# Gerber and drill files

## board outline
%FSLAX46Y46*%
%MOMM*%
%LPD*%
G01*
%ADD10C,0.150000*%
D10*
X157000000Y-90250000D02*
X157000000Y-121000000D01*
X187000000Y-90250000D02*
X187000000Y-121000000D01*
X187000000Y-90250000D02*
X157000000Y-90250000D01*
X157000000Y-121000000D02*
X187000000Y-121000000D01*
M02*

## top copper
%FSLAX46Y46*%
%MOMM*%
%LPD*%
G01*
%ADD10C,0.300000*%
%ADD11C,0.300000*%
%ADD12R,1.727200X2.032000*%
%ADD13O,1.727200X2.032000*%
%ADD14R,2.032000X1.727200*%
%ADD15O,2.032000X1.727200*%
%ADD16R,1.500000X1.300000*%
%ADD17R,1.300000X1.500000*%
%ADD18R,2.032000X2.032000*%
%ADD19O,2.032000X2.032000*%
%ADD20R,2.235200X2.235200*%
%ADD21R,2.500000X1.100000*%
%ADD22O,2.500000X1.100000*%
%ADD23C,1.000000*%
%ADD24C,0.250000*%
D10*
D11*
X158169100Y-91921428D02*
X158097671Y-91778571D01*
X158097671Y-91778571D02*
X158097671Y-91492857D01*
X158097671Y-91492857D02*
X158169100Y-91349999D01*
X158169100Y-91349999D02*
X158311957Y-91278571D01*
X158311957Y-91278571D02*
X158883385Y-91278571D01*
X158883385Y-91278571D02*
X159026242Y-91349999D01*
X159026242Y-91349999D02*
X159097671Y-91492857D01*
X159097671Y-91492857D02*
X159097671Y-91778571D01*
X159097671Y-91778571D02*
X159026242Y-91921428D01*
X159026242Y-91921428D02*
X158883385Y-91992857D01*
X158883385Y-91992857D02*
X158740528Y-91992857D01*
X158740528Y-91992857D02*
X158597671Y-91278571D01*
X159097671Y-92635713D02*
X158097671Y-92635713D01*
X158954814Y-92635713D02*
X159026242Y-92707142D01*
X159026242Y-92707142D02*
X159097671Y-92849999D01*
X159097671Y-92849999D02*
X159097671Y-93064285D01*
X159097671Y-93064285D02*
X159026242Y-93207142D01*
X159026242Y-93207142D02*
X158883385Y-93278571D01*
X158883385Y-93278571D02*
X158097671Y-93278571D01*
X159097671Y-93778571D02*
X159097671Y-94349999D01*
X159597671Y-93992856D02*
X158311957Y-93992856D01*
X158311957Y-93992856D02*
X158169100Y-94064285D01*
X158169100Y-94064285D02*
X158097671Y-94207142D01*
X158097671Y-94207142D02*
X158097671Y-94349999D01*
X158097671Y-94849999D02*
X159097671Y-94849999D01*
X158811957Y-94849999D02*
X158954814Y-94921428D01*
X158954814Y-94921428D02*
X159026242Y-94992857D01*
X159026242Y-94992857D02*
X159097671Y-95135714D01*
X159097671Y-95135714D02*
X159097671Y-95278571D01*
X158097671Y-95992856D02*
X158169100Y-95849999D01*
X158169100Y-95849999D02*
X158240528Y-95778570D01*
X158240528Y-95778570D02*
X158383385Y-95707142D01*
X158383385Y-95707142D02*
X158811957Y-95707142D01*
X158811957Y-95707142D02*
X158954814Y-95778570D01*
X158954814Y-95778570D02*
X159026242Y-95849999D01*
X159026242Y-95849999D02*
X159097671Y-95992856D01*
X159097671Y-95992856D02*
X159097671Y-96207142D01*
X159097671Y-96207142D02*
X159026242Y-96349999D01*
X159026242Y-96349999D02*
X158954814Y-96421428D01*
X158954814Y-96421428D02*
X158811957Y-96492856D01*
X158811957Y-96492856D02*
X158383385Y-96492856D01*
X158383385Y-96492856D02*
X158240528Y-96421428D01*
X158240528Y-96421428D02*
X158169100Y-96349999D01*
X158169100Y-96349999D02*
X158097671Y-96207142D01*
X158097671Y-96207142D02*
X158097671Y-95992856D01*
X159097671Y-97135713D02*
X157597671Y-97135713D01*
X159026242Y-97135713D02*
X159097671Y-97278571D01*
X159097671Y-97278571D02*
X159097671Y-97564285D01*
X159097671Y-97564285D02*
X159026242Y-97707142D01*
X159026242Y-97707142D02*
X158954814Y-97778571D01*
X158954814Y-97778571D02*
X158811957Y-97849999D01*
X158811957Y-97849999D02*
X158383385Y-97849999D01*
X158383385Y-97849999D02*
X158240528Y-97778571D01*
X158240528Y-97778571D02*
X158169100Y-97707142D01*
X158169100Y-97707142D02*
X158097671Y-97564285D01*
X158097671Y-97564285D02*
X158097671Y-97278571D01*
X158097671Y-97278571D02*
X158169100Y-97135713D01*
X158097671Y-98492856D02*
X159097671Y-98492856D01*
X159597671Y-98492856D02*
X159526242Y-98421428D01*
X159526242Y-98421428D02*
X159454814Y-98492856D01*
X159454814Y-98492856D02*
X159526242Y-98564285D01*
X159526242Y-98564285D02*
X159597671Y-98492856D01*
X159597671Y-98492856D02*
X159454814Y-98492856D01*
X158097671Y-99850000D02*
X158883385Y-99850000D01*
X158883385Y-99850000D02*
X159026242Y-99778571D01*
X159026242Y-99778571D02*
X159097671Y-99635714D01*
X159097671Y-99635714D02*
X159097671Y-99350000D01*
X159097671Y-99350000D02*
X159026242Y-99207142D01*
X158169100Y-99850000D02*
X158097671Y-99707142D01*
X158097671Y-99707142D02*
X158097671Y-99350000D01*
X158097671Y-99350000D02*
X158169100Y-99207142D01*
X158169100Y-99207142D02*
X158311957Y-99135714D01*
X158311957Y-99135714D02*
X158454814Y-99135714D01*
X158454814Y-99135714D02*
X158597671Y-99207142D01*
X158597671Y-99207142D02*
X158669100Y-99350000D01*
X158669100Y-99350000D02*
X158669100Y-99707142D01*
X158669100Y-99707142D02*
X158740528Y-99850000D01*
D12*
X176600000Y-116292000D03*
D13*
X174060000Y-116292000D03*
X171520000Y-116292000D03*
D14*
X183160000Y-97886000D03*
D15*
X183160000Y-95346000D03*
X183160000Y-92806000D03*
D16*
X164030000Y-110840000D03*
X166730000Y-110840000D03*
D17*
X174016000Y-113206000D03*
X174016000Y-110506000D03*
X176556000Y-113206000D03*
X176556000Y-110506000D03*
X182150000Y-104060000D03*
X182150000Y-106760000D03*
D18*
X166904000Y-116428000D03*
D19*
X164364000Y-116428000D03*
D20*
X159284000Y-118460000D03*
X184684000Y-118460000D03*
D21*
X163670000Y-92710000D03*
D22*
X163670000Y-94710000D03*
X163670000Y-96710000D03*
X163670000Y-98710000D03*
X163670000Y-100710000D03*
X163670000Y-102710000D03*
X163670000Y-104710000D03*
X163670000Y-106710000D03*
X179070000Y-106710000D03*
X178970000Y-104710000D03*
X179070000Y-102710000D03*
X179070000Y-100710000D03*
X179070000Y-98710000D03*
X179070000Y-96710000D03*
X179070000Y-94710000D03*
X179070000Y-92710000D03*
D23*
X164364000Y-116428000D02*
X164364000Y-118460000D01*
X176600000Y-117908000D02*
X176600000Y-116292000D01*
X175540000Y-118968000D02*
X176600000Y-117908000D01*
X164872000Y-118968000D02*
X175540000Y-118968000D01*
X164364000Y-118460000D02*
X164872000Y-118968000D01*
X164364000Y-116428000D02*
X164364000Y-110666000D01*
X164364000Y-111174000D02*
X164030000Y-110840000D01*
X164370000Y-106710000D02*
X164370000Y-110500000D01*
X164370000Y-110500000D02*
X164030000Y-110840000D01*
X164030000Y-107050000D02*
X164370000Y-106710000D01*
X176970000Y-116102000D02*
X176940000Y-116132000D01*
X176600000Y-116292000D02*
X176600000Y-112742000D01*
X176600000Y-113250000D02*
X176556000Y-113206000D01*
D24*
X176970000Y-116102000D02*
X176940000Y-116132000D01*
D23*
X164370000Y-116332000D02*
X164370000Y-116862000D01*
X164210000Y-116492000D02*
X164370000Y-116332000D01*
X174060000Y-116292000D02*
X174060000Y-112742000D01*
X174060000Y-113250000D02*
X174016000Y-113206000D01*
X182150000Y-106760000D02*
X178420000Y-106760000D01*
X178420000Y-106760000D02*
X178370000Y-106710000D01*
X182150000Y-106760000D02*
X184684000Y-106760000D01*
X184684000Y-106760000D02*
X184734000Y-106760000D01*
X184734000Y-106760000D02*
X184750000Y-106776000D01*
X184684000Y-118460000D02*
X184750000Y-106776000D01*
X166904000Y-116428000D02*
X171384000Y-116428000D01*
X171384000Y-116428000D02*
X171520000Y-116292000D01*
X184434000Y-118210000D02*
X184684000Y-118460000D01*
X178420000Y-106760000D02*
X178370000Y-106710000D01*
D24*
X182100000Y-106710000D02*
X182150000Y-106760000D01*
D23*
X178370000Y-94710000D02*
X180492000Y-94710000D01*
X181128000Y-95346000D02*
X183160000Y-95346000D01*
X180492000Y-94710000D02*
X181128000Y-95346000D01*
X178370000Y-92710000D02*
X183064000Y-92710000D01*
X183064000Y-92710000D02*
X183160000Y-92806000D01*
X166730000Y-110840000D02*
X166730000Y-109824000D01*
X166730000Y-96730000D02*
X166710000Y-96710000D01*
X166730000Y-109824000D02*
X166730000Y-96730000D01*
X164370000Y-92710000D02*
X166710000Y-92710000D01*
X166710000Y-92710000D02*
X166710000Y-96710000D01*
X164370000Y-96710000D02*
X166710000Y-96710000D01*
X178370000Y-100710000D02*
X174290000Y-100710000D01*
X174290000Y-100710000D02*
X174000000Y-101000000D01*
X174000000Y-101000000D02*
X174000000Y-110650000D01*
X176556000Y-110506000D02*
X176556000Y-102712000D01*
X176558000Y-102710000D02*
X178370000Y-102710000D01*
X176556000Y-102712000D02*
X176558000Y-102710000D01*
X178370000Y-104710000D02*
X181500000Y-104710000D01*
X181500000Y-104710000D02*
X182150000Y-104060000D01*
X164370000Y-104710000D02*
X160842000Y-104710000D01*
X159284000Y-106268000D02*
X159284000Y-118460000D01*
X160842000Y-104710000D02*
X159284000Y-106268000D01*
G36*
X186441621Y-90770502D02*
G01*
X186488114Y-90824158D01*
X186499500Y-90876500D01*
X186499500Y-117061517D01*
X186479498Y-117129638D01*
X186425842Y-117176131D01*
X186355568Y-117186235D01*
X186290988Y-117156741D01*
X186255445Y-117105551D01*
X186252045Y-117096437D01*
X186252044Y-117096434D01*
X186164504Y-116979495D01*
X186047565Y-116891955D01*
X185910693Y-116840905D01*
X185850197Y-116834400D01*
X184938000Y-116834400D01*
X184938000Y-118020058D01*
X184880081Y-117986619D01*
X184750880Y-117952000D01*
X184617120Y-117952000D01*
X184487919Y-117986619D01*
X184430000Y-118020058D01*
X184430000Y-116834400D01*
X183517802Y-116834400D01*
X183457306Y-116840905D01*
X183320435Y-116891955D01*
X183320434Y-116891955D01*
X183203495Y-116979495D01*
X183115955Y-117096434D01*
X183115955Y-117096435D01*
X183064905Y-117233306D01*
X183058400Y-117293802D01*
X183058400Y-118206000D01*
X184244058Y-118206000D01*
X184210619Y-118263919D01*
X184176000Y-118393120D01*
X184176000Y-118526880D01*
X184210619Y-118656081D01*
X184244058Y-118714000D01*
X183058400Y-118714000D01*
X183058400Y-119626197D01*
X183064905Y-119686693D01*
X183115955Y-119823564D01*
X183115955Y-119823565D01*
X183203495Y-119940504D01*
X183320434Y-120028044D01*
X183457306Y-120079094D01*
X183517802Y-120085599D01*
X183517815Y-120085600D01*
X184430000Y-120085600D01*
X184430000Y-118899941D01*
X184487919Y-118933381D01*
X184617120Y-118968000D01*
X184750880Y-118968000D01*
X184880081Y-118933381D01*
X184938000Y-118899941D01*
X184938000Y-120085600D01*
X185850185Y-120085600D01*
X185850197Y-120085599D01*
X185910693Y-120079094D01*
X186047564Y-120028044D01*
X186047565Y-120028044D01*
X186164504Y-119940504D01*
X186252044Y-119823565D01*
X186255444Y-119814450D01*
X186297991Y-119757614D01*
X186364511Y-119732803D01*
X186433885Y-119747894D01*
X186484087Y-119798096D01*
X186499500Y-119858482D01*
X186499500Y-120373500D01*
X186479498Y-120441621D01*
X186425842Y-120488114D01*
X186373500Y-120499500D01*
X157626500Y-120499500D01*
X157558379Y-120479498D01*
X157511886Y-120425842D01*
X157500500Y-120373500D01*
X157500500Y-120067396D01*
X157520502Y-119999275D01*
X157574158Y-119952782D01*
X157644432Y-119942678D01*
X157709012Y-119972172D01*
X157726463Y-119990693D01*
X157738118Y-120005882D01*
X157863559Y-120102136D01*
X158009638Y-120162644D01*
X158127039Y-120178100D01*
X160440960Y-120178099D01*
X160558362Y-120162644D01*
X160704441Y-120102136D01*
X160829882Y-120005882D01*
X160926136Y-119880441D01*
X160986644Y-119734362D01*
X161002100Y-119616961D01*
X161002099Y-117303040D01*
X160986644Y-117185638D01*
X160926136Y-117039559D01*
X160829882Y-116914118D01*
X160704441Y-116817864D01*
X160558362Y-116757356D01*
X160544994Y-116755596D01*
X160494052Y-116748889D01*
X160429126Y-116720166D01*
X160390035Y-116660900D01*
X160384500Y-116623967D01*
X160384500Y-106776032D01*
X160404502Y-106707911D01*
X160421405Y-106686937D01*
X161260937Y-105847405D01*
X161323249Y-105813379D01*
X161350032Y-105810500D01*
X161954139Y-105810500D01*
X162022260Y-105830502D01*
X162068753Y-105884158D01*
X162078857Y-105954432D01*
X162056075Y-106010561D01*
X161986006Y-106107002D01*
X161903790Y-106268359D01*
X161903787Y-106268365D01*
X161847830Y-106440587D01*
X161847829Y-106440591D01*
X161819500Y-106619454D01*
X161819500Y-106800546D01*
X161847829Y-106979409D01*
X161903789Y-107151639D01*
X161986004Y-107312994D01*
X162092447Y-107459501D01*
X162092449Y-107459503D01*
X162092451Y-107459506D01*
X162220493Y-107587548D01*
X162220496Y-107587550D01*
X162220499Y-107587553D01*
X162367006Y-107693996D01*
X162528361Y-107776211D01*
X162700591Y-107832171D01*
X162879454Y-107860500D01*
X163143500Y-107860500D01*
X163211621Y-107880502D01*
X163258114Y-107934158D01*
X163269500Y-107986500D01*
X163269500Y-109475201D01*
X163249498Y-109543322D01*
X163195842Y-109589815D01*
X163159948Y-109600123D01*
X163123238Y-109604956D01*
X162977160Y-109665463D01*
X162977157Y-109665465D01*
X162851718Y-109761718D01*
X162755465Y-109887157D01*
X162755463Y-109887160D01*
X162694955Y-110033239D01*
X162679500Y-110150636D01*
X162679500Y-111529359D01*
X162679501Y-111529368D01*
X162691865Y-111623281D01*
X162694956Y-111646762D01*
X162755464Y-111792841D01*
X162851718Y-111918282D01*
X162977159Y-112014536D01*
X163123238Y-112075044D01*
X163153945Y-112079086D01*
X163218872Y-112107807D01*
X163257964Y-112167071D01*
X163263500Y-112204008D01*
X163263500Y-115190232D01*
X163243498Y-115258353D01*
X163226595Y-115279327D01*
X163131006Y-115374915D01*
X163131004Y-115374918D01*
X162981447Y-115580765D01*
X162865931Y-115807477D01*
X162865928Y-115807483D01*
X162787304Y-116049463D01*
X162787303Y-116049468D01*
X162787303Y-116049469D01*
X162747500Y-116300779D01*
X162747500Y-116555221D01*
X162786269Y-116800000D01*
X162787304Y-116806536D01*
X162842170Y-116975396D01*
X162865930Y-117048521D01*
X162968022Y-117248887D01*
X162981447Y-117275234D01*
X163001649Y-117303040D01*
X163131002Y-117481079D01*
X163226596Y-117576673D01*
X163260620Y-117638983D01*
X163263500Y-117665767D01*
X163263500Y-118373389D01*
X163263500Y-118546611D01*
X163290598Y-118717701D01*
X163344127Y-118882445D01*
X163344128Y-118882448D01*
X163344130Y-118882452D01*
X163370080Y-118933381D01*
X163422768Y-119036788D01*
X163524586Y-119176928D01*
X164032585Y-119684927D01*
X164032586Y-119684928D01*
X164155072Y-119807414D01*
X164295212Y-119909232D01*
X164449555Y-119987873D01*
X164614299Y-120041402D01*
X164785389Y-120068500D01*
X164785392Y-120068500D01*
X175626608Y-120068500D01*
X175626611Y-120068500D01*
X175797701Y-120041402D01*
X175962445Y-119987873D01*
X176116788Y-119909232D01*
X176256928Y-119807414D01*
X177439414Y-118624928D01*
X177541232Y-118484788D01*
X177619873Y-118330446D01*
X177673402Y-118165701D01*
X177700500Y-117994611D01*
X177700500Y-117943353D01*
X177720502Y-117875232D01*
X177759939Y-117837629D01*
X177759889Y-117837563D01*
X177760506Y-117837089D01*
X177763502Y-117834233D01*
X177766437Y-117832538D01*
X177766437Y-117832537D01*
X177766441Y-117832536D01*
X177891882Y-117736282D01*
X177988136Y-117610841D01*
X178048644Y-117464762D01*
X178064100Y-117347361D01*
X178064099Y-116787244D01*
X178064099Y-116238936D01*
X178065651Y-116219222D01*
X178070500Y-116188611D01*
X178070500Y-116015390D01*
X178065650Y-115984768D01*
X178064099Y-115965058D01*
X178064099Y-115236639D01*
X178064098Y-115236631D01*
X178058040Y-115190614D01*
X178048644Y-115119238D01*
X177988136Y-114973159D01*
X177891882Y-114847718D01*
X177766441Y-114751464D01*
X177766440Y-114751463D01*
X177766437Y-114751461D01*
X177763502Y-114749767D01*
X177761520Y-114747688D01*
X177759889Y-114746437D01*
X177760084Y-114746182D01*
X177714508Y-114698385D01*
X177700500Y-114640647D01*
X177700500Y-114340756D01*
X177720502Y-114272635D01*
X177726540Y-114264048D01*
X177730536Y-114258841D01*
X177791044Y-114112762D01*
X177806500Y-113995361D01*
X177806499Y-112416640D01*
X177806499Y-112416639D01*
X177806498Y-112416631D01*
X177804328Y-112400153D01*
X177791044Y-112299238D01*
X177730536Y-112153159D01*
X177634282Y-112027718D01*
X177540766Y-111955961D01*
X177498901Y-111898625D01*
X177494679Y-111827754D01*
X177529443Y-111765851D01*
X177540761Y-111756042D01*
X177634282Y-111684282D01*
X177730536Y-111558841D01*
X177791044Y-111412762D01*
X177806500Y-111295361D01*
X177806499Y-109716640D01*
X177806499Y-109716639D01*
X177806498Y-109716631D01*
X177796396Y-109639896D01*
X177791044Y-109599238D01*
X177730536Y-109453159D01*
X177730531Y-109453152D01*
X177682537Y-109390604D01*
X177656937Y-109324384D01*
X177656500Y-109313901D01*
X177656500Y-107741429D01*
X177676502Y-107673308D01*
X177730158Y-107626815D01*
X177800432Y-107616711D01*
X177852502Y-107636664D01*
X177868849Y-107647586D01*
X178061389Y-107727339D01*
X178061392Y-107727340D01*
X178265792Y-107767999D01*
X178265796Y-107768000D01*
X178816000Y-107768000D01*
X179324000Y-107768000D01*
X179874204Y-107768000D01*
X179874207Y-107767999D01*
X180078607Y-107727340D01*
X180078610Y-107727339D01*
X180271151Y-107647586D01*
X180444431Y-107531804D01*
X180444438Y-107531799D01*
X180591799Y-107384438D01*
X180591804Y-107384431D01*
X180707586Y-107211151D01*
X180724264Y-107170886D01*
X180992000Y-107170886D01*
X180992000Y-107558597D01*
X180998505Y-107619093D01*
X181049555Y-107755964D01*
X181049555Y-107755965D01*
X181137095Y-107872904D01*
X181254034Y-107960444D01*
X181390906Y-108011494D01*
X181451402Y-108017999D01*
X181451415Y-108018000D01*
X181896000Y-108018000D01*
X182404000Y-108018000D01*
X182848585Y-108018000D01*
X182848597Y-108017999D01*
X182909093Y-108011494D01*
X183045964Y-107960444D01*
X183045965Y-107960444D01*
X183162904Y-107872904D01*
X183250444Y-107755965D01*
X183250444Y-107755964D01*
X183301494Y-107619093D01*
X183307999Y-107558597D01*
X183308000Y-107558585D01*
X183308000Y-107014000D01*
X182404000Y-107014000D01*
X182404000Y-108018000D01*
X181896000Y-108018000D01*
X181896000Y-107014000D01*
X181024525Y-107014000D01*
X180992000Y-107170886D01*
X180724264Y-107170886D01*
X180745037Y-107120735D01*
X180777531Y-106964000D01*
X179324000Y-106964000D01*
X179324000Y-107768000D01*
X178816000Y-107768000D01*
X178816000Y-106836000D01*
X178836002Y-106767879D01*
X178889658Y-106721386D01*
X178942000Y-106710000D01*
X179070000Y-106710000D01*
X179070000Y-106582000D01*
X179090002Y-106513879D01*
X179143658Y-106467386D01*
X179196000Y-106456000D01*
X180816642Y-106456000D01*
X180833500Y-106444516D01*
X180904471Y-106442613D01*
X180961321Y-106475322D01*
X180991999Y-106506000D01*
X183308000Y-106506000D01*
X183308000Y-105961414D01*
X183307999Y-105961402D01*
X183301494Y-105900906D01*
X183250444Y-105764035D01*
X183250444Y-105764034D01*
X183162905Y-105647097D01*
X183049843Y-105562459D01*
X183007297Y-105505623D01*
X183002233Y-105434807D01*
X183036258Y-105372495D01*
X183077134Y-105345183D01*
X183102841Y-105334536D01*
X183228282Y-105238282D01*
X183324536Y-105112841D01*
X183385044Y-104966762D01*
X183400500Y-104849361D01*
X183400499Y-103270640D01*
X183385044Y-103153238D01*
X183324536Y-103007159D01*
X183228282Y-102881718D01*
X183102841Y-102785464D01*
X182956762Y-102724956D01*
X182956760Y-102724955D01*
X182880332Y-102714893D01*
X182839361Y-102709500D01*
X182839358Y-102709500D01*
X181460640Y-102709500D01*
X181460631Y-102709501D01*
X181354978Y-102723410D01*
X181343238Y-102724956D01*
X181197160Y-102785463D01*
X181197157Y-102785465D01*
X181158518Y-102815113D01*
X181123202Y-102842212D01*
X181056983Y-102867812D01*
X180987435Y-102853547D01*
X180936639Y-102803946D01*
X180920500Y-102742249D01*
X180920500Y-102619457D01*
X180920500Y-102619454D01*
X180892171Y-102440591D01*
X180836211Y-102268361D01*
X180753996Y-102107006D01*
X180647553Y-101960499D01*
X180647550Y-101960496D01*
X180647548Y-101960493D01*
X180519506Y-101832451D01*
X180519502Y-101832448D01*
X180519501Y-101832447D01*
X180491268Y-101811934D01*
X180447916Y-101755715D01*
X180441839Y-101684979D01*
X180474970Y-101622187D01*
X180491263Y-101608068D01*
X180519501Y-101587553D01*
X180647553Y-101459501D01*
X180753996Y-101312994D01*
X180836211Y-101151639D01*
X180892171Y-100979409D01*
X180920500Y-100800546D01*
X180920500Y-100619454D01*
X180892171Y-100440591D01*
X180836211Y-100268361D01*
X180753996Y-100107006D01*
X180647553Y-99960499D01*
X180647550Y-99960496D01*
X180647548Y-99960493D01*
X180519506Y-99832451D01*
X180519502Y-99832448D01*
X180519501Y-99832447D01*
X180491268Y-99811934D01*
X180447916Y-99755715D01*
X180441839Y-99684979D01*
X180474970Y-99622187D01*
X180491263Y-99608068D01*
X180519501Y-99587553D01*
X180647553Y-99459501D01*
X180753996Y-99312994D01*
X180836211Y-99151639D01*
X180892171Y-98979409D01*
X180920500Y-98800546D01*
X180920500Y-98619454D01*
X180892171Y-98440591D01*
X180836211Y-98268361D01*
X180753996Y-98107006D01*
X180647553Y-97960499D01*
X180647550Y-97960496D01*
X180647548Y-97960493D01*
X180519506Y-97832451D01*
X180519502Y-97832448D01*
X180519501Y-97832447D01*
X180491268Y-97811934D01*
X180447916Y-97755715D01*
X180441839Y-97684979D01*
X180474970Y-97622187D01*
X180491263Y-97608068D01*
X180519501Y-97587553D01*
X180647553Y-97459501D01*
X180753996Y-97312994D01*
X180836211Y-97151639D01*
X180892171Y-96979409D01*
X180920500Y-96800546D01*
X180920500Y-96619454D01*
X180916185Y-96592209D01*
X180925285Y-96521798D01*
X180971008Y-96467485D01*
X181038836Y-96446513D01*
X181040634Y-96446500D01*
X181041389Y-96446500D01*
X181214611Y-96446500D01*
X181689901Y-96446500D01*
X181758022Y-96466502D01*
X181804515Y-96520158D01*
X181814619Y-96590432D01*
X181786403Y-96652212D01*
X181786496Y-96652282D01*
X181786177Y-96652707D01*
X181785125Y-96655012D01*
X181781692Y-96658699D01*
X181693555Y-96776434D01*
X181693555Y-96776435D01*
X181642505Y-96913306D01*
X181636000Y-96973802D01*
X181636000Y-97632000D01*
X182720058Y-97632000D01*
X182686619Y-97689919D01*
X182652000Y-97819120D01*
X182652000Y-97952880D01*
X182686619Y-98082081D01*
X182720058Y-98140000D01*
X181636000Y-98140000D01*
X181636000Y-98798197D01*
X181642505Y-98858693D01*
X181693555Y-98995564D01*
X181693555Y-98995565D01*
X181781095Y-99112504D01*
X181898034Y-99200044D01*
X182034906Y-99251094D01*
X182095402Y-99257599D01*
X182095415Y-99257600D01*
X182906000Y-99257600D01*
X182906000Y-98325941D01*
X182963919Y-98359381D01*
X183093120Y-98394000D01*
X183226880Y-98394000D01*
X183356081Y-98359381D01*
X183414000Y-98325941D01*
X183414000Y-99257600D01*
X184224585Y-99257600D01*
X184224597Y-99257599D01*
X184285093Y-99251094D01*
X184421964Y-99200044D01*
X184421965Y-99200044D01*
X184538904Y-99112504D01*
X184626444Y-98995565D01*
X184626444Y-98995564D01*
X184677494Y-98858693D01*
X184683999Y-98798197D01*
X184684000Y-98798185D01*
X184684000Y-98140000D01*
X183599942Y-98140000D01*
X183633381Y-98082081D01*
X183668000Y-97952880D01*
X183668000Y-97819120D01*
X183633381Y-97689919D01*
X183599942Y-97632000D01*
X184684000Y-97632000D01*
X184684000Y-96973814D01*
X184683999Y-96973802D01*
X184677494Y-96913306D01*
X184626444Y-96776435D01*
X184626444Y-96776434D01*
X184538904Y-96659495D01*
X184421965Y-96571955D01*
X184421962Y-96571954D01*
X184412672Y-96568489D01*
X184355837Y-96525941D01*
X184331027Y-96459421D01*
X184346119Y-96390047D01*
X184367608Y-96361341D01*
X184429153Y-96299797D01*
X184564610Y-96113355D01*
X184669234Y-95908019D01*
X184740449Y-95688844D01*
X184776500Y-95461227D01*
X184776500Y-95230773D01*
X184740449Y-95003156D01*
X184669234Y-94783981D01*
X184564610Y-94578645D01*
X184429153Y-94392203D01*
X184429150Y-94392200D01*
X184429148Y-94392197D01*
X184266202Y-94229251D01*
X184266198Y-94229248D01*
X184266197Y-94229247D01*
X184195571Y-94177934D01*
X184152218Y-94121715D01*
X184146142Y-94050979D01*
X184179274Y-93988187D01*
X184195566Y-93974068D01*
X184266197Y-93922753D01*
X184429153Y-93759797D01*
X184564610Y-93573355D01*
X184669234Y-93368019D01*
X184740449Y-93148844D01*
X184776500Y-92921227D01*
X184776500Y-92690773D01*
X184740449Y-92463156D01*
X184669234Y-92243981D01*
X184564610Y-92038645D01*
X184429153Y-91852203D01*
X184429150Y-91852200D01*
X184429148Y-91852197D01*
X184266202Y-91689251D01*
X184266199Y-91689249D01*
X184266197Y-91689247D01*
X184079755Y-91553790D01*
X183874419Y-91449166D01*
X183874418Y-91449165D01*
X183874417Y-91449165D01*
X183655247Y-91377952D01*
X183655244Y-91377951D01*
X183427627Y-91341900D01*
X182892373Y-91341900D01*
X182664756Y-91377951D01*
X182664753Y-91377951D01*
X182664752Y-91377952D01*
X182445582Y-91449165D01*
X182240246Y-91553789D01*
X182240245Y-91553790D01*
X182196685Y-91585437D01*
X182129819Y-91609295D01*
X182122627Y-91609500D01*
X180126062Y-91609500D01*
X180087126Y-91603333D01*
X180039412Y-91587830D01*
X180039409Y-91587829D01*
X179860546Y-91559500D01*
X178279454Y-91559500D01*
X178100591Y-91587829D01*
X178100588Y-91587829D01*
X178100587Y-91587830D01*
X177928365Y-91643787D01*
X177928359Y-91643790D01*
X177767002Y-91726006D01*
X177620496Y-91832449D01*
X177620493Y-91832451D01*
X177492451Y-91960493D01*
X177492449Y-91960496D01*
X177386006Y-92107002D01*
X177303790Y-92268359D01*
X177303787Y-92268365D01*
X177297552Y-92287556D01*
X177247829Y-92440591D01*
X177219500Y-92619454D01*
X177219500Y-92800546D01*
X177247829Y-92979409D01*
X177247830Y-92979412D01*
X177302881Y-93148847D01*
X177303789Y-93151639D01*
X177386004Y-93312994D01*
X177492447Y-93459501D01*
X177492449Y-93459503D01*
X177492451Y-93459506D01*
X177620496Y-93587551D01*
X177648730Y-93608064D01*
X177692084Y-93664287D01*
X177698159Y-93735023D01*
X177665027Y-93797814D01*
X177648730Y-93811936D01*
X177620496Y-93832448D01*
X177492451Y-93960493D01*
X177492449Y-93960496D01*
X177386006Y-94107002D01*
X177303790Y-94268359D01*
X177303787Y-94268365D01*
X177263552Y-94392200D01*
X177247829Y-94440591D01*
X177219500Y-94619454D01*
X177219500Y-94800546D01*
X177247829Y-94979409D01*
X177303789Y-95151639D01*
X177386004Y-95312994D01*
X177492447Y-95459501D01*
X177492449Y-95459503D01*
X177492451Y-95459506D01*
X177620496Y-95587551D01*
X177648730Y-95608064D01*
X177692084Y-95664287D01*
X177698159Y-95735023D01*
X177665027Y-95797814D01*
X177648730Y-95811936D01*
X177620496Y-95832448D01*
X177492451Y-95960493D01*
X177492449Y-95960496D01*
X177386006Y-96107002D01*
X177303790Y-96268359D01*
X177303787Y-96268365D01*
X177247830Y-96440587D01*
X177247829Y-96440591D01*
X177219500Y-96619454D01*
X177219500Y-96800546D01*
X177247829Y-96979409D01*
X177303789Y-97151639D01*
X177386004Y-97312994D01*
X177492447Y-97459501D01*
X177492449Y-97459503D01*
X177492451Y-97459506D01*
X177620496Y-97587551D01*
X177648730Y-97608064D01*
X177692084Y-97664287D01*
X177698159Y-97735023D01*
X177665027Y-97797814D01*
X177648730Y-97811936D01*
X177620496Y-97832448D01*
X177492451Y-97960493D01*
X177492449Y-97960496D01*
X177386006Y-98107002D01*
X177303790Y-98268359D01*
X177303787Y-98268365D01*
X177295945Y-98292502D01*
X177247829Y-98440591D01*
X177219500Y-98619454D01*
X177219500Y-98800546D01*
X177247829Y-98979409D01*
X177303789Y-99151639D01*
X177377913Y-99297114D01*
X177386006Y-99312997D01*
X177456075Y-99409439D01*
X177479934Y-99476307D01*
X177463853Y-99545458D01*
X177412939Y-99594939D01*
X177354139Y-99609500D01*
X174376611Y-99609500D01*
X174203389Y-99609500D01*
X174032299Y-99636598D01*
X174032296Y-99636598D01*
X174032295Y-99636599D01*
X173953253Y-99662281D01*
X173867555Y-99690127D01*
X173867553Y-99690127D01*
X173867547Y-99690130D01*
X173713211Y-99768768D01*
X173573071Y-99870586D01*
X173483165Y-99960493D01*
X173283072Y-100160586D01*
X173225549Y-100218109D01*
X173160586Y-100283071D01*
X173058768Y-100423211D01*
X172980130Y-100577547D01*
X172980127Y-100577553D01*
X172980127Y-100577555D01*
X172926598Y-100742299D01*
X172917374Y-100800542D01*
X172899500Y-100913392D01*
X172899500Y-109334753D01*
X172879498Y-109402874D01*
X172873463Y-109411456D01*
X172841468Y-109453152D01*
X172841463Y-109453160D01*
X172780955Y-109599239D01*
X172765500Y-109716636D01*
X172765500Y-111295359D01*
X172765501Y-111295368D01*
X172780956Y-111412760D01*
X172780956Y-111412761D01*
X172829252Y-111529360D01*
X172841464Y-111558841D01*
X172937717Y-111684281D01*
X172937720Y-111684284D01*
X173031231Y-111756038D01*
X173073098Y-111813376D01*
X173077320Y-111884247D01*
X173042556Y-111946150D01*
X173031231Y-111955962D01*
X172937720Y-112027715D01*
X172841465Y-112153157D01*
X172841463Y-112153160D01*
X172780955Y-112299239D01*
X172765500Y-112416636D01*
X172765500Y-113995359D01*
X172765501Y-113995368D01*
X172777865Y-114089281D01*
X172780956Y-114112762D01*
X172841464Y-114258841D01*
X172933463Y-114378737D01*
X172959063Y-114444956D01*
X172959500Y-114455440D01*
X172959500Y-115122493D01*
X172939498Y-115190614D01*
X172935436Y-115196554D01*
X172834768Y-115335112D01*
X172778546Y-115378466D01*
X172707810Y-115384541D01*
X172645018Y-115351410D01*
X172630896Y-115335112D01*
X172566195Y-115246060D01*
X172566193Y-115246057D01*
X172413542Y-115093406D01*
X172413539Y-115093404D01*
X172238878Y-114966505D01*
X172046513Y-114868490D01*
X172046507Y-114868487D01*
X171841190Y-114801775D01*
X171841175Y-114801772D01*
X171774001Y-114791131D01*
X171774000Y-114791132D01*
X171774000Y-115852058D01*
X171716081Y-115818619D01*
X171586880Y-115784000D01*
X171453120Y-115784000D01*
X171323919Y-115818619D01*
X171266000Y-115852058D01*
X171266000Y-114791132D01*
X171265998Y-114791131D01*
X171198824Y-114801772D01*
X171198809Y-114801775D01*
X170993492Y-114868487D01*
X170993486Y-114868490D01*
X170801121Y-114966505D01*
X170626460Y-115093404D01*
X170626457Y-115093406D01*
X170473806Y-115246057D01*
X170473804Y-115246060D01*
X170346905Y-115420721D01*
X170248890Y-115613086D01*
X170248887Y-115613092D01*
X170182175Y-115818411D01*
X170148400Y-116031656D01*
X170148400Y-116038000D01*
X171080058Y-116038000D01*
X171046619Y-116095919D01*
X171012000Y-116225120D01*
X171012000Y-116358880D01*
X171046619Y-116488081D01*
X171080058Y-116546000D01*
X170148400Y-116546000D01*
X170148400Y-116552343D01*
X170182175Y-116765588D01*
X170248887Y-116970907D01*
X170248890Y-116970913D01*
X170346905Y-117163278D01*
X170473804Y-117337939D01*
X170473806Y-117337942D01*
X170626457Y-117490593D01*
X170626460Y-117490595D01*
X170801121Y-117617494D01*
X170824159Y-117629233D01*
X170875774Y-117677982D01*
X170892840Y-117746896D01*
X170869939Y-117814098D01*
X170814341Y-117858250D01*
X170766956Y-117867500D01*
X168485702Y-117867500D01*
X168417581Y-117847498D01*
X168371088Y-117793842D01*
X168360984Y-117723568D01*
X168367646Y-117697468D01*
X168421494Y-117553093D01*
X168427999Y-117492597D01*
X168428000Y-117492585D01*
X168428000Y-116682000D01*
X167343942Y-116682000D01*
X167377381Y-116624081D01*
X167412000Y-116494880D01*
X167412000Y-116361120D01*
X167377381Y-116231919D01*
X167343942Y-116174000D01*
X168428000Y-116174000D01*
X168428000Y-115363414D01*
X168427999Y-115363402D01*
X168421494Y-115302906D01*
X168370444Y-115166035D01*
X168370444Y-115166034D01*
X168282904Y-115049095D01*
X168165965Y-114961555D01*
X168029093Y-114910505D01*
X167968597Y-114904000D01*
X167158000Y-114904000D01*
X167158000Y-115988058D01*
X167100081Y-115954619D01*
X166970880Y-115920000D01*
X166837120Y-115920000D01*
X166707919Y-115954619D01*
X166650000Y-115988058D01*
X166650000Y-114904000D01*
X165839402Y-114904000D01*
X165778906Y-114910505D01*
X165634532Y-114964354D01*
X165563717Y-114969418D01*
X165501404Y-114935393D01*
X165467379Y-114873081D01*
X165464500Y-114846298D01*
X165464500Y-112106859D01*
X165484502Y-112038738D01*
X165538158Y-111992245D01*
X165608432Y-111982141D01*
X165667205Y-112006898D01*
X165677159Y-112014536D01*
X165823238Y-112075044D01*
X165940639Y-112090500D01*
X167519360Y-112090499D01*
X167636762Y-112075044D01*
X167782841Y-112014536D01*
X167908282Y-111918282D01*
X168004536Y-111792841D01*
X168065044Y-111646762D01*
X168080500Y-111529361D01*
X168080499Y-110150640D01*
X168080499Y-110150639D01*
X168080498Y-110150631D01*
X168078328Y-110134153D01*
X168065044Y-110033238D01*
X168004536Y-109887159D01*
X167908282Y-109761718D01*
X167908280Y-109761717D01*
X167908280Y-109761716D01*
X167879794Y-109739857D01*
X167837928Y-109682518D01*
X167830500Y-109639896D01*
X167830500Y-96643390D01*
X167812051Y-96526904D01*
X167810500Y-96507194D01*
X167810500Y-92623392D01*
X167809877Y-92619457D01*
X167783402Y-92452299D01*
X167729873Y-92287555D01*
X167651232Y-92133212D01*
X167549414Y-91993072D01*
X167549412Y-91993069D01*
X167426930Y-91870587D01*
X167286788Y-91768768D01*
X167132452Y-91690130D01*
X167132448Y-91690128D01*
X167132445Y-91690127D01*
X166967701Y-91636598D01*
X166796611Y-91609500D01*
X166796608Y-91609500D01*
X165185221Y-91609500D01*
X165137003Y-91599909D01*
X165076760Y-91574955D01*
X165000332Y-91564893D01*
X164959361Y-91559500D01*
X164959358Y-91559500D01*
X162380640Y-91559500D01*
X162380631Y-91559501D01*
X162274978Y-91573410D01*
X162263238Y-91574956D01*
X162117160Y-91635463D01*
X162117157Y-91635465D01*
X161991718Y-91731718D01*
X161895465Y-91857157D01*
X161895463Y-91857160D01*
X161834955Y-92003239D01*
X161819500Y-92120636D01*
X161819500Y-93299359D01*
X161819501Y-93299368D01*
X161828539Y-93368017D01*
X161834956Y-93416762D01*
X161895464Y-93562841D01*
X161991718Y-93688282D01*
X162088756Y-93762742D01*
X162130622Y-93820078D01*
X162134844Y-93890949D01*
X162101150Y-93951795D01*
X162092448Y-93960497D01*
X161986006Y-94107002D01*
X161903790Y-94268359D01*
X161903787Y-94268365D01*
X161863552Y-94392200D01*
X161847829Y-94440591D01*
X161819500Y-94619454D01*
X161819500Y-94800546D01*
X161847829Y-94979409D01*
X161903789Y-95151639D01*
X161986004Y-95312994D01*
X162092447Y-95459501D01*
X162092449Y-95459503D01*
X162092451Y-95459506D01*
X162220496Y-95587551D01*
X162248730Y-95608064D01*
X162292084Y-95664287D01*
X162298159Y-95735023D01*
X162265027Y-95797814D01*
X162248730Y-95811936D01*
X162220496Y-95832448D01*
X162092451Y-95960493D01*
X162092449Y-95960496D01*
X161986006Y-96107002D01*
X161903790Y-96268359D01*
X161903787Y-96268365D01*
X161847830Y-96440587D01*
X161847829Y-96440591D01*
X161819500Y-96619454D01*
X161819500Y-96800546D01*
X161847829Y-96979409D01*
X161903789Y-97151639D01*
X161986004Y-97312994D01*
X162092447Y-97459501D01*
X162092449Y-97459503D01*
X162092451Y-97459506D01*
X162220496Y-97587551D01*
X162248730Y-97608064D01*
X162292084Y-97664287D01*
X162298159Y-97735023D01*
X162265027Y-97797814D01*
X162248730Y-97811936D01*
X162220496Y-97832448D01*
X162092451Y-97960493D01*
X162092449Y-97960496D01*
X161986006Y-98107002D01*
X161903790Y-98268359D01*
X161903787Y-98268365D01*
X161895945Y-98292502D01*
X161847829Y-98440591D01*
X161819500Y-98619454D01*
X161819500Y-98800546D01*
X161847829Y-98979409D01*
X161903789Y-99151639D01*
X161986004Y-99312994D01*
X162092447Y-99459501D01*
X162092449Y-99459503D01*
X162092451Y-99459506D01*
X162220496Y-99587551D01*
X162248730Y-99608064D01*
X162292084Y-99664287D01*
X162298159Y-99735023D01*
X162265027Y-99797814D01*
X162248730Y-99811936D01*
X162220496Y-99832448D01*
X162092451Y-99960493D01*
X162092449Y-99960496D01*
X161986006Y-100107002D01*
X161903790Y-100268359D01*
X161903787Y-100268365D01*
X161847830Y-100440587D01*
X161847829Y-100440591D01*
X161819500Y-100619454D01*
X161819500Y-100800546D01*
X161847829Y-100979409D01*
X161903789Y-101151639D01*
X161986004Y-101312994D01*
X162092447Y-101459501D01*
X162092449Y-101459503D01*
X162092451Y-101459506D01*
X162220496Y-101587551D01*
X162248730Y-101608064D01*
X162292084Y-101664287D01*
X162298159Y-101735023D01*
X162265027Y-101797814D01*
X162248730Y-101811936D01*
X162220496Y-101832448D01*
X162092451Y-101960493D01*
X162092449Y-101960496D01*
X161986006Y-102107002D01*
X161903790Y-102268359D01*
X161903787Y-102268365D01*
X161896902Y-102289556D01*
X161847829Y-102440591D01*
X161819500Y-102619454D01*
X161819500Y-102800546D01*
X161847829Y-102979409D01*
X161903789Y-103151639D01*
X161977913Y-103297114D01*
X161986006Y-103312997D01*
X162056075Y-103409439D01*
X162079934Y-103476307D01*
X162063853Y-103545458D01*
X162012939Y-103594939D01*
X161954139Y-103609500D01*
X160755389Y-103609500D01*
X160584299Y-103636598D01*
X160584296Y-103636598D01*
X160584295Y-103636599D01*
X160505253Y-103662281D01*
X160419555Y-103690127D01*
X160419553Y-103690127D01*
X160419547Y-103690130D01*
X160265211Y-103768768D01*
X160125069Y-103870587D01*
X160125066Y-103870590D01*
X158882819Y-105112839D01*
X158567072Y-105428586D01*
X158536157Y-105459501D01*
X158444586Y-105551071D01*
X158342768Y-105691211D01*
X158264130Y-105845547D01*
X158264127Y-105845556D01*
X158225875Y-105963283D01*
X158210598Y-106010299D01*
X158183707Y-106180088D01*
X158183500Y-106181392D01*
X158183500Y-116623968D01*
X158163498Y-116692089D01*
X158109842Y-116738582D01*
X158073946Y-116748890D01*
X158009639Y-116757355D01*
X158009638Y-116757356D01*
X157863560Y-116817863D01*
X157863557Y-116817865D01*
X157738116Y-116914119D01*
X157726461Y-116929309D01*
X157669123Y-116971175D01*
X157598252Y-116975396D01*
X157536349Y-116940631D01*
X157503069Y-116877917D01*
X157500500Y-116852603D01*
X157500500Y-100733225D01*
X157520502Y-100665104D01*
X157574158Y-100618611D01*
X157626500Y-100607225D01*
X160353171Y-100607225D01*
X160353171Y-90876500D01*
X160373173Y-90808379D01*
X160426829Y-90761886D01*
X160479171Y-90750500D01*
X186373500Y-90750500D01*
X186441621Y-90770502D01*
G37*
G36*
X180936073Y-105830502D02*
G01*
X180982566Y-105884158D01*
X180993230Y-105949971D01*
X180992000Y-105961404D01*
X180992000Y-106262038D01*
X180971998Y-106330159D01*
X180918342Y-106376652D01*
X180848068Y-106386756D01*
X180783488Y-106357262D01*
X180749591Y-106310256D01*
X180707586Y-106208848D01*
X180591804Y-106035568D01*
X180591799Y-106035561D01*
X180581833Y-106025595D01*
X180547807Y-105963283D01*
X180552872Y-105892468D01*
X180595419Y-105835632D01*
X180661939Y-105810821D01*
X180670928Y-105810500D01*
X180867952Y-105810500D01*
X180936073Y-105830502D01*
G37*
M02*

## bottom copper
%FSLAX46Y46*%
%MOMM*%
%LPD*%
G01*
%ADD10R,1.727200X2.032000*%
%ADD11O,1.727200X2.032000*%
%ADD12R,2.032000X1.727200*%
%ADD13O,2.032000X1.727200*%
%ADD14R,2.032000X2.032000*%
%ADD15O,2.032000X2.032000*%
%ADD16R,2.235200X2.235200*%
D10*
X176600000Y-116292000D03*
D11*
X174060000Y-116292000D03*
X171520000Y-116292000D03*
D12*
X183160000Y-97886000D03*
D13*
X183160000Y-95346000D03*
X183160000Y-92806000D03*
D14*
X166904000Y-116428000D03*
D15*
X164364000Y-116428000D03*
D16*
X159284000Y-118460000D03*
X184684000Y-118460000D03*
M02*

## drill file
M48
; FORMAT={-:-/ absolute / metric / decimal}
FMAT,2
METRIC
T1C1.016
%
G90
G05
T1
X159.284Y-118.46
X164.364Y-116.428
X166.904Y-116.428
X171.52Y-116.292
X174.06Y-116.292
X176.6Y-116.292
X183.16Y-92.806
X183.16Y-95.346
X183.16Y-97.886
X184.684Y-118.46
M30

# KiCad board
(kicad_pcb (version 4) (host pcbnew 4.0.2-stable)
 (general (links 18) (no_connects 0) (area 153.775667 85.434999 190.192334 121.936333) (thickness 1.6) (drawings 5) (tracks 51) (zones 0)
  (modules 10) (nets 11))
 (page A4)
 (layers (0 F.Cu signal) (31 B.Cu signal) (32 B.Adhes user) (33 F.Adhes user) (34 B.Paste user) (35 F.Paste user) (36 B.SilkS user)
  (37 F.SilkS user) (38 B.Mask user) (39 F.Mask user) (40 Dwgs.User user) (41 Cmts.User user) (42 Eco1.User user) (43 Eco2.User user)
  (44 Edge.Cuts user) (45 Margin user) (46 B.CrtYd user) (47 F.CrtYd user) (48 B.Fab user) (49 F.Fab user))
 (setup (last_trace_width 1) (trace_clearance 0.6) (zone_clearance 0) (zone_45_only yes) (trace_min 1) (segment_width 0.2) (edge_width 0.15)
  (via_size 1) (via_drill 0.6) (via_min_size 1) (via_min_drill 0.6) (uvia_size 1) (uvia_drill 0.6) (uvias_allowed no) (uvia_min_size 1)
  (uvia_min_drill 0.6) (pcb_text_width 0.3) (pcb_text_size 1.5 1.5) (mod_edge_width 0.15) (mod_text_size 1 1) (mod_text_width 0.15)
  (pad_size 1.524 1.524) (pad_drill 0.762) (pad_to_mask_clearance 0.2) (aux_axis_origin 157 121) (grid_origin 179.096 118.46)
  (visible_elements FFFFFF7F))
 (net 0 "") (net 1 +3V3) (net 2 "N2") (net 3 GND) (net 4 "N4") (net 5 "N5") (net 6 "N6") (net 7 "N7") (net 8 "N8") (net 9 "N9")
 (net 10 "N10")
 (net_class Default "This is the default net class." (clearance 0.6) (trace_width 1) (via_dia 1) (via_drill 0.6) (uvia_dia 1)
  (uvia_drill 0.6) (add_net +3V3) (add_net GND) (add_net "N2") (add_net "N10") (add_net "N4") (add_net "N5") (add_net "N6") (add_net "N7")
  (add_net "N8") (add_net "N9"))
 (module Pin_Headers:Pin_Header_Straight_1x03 (layer F.Cu) (at 176.6 116.292 270)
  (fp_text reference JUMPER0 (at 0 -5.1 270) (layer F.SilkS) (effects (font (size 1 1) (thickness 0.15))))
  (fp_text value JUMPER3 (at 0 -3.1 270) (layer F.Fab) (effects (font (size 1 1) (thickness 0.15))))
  (pad 1 thru_hole rect (at 0 0 270) (size 2.032 1.7272) (drill 1.016) (layers *.Cu *.Mask F.SilkS) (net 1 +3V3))
  (pad 2 thru_hole oval (at 0 2.54 270) (size 2.032 1.7272) (drill 1.016) (layers *.Cu *.Mask F.SilkS) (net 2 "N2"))
  (pad 3 thru_hole oval (at 0 5.08 270) (size 2.032 1.7272) (drill 1.016) (layers *.Cu *.Mask F.SilkS) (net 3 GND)))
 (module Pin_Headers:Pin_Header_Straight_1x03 (layer F.Cu) (at 183.16 97.886 180)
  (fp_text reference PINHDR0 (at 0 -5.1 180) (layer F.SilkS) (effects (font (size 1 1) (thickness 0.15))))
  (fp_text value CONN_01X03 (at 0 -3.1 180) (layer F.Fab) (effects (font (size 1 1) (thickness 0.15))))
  (pad 1 thru_hole rect (at 0 0 180) (size 2.032 1.7272) (drill 1.016) (layers *.Cu *.Mask F.SilkS) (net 3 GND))
  (pad 2 thru_hole oval (at 0 2.54 180) (size 2.032 1.7272) (drill 1.016) (layers *.Cu *.Mask F.SilkS) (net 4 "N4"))
  (pad 3 thru_hole oval (at 0 5.08 180) (size 2.032 1.7272) (drill 1.016) (layers *.Cu *.Mask F.SilkS) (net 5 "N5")))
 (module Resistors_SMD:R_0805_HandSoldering (layer F.Cu) (at 165.38 110.84)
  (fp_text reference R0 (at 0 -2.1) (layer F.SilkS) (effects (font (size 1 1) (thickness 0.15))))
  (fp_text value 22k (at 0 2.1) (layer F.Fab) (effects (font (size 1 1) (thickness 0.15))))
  (pad 1 smd rect (at -1.35 0) (size 1.5 1.3) (layers F.Cu F.Paste F.Mask) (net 1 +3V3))
  (pad 2 smd rect (at 1.35 0) (size 1.5 1.3) (layers F.Cu F.Paste F.Mask) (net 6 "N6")))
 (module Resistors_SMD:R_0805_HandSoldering (layer F.Cu) (at 174.016 111.856 90)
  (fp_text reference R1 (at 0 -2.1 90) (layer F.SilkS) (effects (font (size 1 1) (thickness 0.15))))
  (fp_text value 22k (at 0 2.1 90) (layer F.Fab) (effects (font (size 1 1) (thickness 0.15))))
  (pad 1 smd rect (at -1.35 0 90) (size 1.5 1.3) (layers F.Cu F.Paste F.Mask) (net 2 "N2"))
  (pad 2 smd rect (at 1.35 0 90) (size 1.5 1.3) (layers F.Cu F.Paste F.Mask) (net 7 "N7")))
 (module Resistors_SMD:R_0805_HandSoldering (layer F.Cu) (at 176.556 111.856 90)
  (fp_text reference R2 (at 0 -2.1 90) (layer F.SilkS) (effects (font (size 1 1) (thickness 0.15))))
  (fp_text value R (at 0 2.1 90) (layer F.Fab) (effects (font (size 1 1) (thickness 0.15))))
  (pad 1 smd rect (at -1.35 0 90) (size 1.5 1.3) (layers F.Cu F.Paste F.Mask) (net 1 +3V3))
  (pad 2 smd rect (at 1.35 0 90) (size 1.5 1.3) (layers F.Cu F.Paste F.Mask) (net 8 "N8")))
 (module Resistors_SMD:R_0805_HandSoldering (layer F.Cu) (at 182.15 105.41 270)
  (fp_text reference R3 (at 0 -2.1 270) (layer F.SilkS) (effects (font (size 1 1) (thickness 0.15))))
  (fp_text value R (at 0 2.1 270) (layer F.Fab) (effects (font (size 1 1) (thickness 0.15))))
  (pad 1 smd rect (at -1.35 0 270) (size 1.5 1.3) (layers F.Cu F.Paste F.Mask) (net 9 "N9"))
  (pad 2 smd rect (at 1.35 0 270) (size 1.5 1.3) (layers F.Cu F.Paste F.Mask) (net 3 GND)))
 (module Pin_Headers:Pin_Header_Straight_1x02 (layer F.Cu) (at 166.904 116.428 270)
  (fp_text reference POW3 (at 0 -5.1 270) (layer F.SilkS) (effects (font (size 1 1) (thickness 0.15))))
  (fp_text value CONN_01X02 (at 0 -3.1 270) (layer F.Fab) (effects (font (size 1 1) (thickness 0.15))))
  (pad 1 thru_hole rect (at 0 0 270) (size 2.032 2.032) (drill 1.016) (layers *.Cu *.Mask F.SilkS) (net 3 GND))
  (pad 2 thru_hole oval (at 0 2.54 270) (size 2.032 2.032) (drill 1.016) (layers *.Cu *.Mask F.SilkS) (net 1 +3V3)))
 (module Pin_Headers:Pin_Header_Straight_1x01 (layer F.Cu) (at 159.284 118.46)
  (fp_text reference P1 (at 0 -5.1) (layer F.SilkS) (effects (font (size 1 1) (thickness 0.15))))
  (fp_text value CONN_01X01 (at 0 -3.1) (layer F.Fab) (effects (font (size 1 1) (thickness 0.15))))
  (pad 1 thru_hole rect (at 0 0) (size 2.2352 2.2352) (drill 1.016) (layers *.Cu *.Mask F.SilkS) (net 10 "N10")))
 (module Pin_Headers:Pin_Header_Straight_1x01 (layer F.Cu) (at 184.684 118.46)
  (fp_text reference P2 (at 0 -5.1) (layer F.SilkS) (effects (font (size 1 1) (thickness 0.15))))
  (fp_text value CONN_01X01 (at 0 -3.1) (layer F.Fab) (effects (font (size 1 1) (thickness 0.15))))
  (pad 1 thru_hole rect (at 0 0) (size 2.2352 2.2352) (drill 1.016) (layers *.Cu *.Mask F.SilkS) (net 3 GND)))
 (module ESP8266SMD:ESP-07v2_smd (layer F.Cu) (at 164.37 92.71)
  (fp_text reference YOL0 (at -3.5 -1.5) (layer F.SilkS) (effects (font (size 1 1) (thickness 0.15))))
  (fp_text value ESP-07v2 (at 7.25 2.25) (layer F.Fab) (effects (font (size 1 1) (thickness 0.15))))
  (pad 1 smd rect (at 0 0) (size 2.5 1.1) (drill (offset -0.7 0)) (layers F.Cu F.Paste F.Mask) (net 6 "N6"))
  (pad 2 smd oval (at 0 2) (size 2.5 1.1) (drill (offset -0.7 0)) (layers F.Cu F.Paste F.Mask))
  (pad 3 smd oval (at 0 4) (size 2.5 1.1) (drill (offset -0.7 0)) (layers F.Cu F.Paste F.Mask) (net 6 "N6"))
  (pad 4 smd oval (at 0 6) (size 2.5 1.1) (drill (offset -0.7 0)) (layers F.Cu F.Paste F.Mask))
  (pad 5 smd oval (at 0 8) (size 2.5 1.1) (drill (offset -0.7 0)) (layers F.Cu F.Paste F.Mask))
  (pad 6 smd oval (at 0 10) (size 2.5 1.1) (drill (offset -0.7 0)) (layers F.Cu F.Paste F.Mask))
  (pad 7 smd oval (at 0 12) (size 2.5 1.1) (drill (offset -0.7 0)) (layers F.Cu F.Paste F.Mask) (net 10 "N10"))
  (pad 8 smd oval (at 0 14) (size 2.5 1.1) (drill (offset -0.7 0)) (layers F.Cu F.Paste F.Mask) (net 1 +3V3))
  (pad 9 smd oval (at 14 14) (size 2.5 1.1) (drill (offset 0.7 0)) (layers F.Cu F.Paste F.Mask) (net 3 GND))
  (pad 10 smd oval (at 14 12) (size 2.5 1.1) (drill (offset 0.6 0)) (layers F.Cu F.Paste F.Mask) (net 9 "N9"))
  (pad 11 smd oval (at 14 10) (size 2.5 1.1) (drill (offset 0.7 0)) (layers F.Cu F.Paste F.Mask) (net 8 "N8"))
  (pad 12 smd oval (at 14 8) (size 2.5 1.1) (drill (offset 0.7 0)) (layers F.Cu F.Paste F.Mask) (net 7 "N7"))
  (pad 13 smd oval (at 14 6) (size 2.5 1.1) (drill (offset 0.7 0)) (layers F.Cu F.Paste F.Mask))
  (pad 14 smd oval (at 14 4) (size 2.5 1.1) (drill (offset 0.7 0)) (layers F.Cu F.Paste F.Mask))
  (pad 15 smd oval (at 14 2) (size 2.5 1.1) (drill (offset 0.7 0)) (layers F.Cu F.Paste F.Mask) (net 4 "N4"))
  (pad 16 smd oval (at 14 0) (size 2.5 1.1) (drill (offset 0.7 0)) (layers F.Cu F.Paste F.Mask) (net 5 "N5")))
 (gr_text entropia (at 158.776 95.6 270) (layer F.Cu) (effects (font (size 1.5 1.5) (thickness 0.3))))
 (gr_line (start 157 90.25) (end 157 121) (angle 90) (layer Edge.Cuts) (width 0.15))
 (gr_line (start 187 90.25) (end 187 121) (angle 90) (layer Edge.Cuts) (width 0.15))
 (gr_line (start 187 90.25) (end 157 90.25) (angle 90) (layer Edge.Cuts) (width 0.15))
 (gr_line (start 157 121) (end 187 121) (angle 90) (layer Edge.Cuts) (width 0.15))
 (segment (start 164.364 116.428) (end 164.364 118.46) (width 1) (layer F.Cu) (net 1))
 (segment (start 176.6 117.908) (end 176.6 116.292) (width 1) (layer F.Cu) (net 1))
 (segment (start 175.54 118.968) (end 176.6 117.908) (width 1) (layer F.Cu) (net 1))
 (segment (start 164.872 118.968) (end 175.54 118.968) (width 1) (layer F.Cu) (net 1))
 (segment (start 164.364 118.46) (end 164.872 118.968) (width 1) (layer F.Cu) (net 1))
 (segment (start 164.364 116.428) (end 164.364 110.666) (width 1) (layer F.Cu) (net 1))
 (segment (start 164.364 111.174) (end 164.03 110.84) (width 1) (layer F.Cu) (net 1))
 (segment (start 164.37 106.71) (end 164.37 110.5) (width 1) (layer F.Cu) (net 1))
 (segment (start 164.37 110.5) (end 164.03 110.84) (width 1) (layer F.Cu) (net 1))
 (segment (start 164.03 107.05) (end 164.37 106.71) (width 1) (layer F.Cu) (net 1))
 (segment (start 176.97 116.102) (end 176.94 116.132) (width 1) (layer F.Cu) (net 1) (status 30))
 (segment (start 176.6 116.292) (end 176.6 112.742) (width 1) (layer F.Cu) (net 1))
 (segment (start 176.6 113.25) (end 176.556 113.206) (width 1) (layer F.Cu) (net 1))
 (segment (start 176.97 116.102) (end 176.94 116.132) (width 0.25) (layer F.Cu) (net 1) (status 30))
 (segment (start 164.37 116.332) (end 164.37 116.862) (width 1) (layer F.Cu) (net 1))
 (segment (start 164.21 116.492) (end 164.37 116.332) (width 1) (layer F.Cu) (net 1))
 (segment (start 174.06 116.292) (end 174.06 112.742) (width 1) (layer F.Cu) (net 2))
 (segment (start 174.06 113.25) (end 174.016 113.206) (width 1) (layer F.Cu) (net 2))
 (segment (start 182.15 106.76) (end 178.42 106.76) (width 1) (layer F.Cu) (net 3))
 (segment (start 178.42 106.76) (end 178.37 106.71) (width 1) (layer F.Cu) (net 3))
 (segment (start 182.15 106.76) (end 184.684 106.76) (width 1) (layer F.Cu) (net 3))
 (segment (start 184.684 106.76) (end 184.734 106.76) (width 1) (layer F.Cu) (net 3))
 (segment (start 184.734 106.76) (end 184.75 106.776) (width 1) (layer F.Cu) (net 3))
 (segment (start 184.684 118.46) (end 184.75 106.776) (width 1) (layer F.Cu) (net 3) (status 10))
 (segment (start 166.904 116.428) (end 171.384 116.428) (width 1) (layer F.Cu) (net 3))
 (segment (start 171.384 116.428) (end 171.52 116.292) (width 1) (layer F.Cu) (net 3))
 (segment (start 184.434 118.21) (end 184.684 118.46) (width 1) (layer F.Cu) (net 3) (status 30))
 (segment (start 178.42 106.76) (end 178.37 106.71) (width 1) (layer F.Cu) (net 3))
 (segment (start 182.1 106.71) (end 182.15 106.76) (width 0.25) (layer F.Cu) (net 3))
 (segment (start 178.37 94.71) (end 180.492 94.71) (width 1) (layer F.Cu) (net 4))
 (segment (start 181.128 95.346) (end 183.16 95.346) (width 1) (layer F.Cu) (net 4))
 (segment (start 180.492 94.71) (end 181.128 95.346) (width 1) (layer F.Cu) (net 4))
 (segment (start 178.37 92.71) (end 183.064 92.71) (width 1) (layer F.Cu) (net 5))
 (segment (start 183.064 92.71) (end 183.16 92.806) (width 1) (layer F.Cu) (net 5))
 (segment (start 166.73 110.84) (end 166.73 109.824) (width 1) (layer F.Cu) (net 6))
 (segment (start 166.73 96.73) (end 166.71 96.71) (width 1) (layer F.Cu) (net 6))
 (segment (start 166.73 109.824) (end 166.73 96.73) (width 1) (layer F.Cu) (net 6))
 (segment (start 164.37 92.71) (end 166.71 92.71) (width 1) (layer F.Cu) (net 6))
 (segment (start 166.71 92.71) (end 166.71 96.71) (width 1) (layer F.Cu) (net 6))
 (segment (start 164.37 96.71) (end 166.71 96.71) (width 1) (layer F.Cu) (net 6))
 (segment (start 178.37 100.71) (end 174.29 100.71) (width 1) (layer F.Cu) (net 7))
 (segment (start 174.29 100.71) (end 174 101) (width 1) (layer F.Cu) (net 7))
 (segment (start 174 101) (end 174 110.65) (width 1) (layer F.Cu) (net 7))
 (segment (start 176.556 110.506) (end 176.556 102.712) (width 1) (layer F.Cu) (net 8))
 (segment (start 176.558 102.71) (end 178.37 102.71) (width 1) (layer F.Cu) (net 8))
 (segment (start 176.556 102.712) (end 176.558 102.71) (width 1) (layer F.Cu) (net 8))
 (segment (start 178.37 104.71) (end 181.5 104.71) (width 1) (layer F.Cu) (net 9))
 (segment (start 181.5 104.71) (end 182.15 104.06) (width 1) (layer F.Cu) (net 9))
 (segment (start 164.37 104.71) (end 160.842 104.71) (width 1) (layer F.Cu) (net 10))
 (segment (start 159.284 106.268) (end 159.284 118.46) (width 1) (layer F.Cu) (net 10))
 (segment (start 160.842 104.71) (end 159.284 106.268) (width 1) (layer F.Cu) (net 10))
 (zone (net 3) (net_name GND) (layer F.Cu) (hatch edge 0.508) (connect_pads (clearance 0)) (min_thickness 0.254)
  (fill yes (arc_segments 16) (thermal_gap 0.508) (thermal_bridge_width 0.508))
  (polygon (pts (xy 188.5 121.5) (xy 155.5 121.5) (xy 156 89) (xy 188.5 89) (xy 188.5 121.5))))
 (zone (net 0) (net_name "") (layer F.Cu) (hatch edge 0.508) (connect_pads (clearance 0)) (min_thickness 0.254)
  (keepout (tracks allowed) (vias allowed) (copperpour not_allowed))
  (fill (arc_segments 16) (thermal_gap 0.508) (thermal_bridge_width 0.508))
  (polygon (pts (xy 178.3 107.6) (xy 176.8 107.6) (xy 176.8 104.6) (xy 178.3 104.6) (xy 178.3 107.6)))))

